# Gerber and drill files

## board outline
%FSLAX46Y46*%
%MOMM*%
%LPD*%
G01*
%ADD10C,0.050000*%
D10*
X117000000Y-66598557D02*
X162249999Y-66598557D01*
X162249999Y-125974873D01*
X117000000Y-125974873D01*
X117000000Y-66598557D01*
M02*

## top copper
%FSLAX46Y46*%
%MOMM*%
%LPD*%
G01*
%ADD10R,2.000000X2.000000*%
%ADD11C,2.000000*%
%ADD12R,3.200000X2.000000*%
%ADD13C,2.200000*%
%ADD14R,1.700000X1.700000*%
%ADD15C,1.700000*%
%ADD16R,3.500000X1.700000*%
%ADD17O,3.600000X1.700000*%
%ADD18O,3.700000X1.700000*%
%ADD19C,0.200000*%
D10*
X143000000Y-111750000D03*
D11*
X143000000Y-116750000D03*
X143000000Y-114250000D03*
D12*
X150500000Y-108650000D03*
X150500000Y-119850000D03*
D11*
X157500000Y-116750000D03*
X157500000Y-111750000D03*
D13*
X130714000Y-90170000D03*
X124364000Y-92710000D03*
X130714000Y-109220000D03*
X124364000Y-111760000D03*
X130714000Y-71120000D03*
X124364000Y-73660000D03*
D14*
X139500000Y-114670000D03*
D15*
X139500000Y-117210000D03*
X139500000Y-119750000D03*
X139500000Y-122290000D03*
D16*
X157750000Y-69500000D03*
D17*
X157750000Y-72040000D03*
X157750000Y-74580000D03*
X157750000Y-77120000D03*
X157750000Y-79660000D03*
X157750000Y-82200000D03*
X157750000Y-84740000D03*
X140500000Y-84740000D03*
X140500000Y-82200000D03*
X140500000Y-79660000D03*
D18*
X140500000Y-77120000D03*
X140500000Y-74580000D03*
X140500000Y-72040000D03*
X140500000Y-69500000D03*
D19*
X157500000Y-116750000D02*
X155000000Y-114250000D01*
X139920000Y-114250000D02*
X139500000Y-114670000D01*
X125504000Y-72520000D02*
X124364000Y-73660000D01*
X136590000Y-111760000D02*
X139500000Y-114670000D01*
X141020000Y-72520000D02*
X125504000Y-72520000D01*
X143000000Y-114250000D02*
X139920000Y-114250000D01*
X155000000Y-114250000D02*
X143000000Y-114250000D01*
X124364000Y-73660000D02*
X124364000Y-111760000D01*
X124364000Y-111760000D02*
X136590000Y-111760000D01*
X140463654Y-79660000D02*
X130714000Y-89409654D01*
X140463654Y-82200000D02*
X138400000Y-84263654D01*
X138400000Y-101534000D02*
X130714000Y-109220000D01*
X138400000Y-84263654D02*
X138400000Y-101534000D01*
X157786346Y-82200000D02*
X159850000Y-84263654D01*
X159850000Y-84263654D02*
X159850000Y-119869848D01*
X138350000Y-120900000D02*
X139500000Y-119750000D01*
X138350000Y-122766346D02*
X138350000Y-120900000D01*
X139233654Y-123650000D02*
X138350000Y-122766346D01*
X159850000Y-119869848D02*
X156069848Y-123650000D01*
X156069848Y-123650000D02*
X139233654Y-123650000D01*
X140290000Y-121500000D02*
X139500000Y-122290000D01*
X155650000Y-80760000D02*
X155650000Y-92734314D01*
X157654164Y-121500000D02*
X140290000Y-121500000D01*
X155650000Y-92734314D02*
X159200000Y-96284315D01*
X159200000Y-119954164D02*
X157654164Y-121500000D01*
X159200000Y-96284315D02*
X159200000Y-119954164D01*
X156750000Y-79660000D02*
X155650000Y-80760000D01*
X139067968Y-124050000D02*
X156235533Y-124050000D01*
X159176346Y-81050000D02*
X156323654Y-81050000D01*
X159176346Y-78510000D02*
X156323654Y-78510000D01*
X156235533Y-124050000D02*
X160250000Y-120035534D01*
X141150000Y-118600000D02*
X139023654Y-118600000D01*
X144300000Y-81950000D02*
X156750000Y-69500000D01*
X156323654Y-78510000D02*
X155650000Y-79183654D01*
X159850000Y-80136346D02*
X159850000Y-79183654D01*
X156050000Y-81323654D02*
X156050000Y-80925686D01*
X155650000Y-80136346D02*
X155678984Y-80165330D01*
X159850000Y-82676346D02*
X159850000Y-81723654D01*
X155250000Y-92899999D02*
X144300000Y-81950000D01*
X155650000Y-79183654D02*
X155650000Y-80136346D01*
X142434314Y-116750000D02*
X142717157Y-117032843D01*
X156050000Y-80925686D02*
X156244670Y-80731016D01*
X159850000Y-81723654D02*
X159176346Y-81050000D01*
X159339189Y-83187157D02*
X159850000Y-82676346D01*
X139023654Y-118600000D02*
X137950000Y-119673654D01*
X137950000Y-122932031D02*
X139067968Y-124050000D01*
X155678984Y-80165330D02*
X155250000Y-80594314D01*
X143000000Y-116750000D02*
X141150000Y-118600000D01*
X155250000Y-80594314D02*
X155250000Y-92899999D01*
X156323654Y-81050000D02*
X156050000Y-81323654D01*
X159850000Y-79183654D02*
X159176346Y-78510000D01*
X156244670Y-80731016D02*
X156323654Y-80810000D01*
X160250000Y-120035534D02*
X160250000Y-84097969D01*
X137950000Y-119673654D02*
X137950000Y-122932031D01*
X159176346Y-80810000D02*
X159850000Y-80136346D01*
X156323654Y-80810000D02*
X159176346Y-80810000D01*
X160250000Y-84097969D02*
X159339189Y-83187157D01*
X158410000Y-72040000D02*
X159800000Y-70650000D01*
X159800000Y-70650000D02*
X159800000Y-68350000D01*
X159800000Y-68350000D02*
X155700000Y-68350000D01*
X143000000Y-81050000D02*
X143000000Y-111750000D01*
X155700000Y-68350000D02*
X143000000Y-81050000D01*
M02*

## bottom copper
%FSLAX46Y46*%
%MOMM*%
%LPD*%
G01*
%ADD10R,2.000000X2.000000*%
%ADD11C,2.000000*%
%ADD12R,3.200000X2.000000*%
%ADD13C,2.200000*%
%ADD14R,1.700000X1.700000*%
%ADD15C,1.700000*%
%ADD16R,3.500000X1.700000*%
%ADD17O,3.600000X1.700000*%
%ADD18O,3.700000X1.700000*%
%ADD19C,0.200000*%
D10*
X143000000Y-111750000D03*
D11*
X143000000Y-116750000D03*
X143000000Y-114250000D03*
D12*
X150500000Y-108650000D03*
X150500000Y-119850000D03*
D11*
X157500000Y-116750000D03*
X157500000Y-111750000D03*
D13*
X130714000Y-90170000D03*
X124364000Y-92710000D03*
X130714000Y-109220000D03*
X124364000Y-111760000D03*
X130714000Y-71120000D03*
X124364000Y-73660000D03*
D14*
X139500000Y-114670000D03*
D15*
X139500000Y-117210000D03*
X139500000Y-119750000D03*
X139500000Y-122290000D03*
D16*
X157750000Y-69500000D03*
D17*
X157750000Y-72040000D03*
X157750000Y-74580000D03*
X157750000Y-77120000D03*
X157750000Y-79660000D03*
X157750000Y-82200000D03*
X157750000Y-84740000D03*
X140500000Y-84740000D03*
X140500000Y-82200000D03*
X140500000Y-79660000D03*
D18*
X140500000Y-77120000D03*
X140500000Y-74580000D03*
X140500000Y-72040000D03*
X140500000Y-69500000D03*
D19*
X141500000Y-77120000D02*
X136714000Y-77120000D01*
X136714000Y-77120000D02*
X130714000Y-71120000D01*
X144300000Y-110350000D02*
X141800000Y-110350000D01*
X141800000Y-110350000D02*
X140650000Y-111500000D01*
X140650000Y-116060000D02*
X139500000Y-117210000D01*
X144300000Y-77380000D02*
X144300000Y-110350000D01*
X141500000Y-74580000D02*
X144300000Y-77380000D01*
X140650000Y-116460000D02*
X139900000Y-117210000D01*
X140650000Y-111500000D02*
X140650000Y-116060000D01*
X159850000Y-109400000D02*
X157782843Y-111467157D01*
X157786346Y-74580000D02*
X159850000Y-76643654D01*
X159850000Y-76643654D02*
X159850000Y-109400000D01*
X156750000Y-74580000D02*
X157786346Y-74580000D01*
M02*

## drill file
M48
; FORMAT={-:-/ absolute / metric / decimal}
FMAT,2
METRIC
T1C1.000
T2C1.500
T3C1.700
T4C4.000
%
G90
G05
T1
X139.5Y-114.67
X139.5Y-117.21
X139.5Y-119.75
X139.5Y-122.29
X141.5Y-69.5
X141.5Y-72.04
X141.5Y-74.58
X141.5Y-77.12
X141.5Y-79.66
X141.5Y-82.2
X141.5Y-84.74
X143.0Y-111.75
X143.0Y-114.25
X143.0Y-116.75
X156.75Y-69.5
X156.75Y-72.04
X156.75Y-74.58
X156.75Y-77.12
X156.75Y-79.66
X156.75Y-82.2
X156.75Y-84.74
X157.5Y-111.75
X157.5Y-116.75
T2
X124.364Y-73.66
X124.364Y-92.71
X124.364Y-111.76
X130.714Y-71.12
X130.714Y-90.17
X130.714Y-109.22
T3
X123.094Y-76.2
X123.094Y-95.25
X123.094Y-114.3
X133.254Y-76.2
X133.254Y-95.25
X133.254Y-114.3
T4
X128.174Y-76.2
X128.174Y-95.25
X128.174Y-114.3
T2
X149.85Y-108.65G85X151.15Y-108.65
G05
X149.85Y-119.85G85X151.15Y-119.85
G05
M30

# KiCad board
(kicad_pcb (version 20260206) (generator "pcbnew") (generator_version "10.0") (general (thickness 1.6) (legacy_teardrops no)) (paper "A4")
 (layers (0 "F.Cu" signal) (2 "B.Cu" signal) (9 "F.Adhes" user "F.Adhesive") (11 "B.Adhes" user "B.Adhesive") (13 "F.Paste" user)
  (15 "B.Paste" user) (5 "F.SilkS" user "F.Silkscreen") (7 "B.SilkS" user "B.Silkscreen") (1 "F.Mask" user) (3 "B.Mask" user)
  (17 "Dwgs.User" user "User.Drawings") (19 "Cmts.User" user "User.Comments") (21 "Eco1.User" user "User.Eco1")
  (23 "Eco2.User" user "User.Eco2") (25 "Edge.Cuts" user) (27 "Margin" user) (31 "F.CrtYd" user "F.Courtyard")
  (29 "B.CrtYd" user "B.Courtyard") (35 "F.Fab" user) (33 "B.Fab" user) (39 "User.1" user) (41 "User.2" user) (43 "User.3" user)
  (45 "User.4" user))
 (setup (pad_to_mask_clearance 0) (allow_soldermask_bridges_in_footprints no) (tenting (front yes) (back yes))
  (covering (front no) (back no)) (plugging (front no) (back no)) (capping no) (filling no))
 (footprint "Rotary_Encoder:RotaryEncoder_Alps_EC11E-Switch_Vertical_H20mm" (layer "F.Cu") (at 143 111.75)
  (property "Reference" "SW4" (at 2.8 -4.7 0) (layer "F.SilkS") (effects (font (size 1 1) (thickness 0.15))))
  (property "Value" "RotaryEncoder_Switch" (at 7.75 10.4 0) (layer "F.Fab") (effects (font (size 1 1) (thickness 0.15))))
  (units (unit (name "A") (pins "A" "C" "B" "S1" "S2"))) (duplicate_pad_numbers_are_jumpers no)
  (pad "A" thru_hole rect (at 0 0) (size 2 2) (drill 1) (layers "*.Cu" "*.Mask") (remove_unused_layers no) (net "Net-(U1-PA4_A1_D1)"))
  (pad "B" thru_hole circle (at 0 5) (size 2 2) (drill 1) (layers "*.Cu" "*.Mask") (remove_unused_layers no) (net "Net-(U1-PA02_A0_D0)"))
  (pad "C" thru_hole circle (at 0 2.5) (size 2 2) (drill 1) (layers "*.Cu" "*.Mask") (remove_unused_layers no) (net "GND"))
  (pad "MP" thru_hole rect (at 7.5 -3.1) (size 3.2 2) (drill oval 2.8 1.5) (layers "*.Cu" "*.Mask") (remove_unused_layers no))
  (pad "MP" thru_hole rect (at 7.5 8.1) (size 3.2 2) (drill oval 2.8 1.5) (layers "*.Cu" "*.Mask") (remove_unused_layers no))
  (pad "S1" thru_hole circle (at 14.5 5) (size 2 2) (drill 1) (layers "*.Cu" "*.Mask") (remove_unused_layers no) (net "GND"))
  (pad "S2" thru_hole circle (at 14.5 0) (size 2 2) (drill 1) (layers "*.Cu" "*.Mask") (remove_unused_layers no) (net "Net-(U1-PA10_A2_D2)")))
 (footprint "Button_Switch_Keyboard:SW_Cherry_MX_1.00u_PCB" (layer "F.Cu") (at 130.714 90.17)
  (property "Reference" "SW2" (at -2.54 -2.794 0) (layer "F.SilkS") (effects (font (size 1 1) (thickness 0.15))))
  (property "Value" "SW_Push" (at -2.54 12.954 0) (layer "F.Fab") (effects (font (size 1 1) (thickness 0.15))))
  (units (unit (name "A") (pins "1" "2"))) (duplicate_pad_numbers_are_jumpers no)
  (pad "" np_thru_hole circle (at -7.62 5.08) (size 1.7 1.7) (drill 1.7) (layers "*.Cu" "*.Mask"))
  (pad "" np_thru_hole circle (at -2.54 5.08) (size 4 4) (drill 4) (layers "*.Cu" "*.Mask"))
  (pad "" np_thru_hole circle (at 2.54 5.08) (size 1.7 1.7) (drill 1.7) (layers "*.Cu" "*.Mask"))
  (pad "1" thru_hole circle (at 0 0) (size 2.2 2.2) (drill 1.5) (layers "*.Cu" "*.Mask") (remove_unused_layers no)
   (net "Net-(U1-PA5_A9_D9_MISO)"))
  (pad "2" thru_hole circle (at -6.35 2.54) (size 2.2 2.2) (drill 1.5) (layers "*.Cu" "*.Mask") (remove_unused_layers no) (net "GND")))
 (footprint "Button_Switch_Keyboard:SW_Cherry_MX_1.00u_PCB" (layer "F.Cu") (at 130.714 109.22)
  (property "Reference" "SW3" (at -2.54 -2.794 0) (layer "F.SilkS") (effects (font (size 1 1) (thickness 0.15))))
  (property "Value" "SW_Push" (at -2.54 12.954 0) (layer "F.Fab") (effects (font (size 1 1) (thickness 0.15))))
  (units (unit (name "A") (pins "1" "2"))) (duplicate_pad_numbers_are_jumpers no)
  (pad "" np_thru_hole circle (at -7.62 5.08) (size 1.7 1.7) (drill 1.7) (layers "*.Cu" "*.Mask"))
  (pad "" np_thru_hole circle (at -2.54 5.08) (size 4 4) (drill 4) (layers "*.Cu" "*.Mask"))
  (pad "" np_thru_hole circle (at 2.54 5.08) (size 1.7 1.7) (drill 1.7) (layers "*.Cu" "*.Mask"))
  (pad "1" thru_hole circle (at 0 0) (size 2.2 2.2) (drill 1.5) (layers "*.Cu" "*.Mask") (remove_unused_layers no)
   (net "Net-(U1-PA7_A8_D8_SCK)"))
  (pad "2" thru_hole circle (at -6.35 2.54) (size 2.2 2.2) (drill 1.5) (layers "*.Cu" "*.Mask") (remove_unused_layers no) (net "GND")))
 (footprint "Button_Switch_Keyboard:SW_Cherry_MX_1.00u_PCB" (layer "F.Cu") (at 130.714 71.12)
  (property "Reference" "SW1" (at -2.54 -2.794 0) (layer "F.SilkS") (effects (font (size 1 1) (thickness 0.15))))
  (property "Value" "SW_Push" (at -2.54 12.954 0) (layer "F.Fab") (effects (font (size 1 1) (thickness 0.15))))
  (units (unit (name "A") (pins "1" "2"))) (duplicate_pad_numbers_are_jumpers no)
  (pad "" np_thru_hole circle (at -7.62 5.08) (size 1.7 1.7) (drill 1.7) (layers "*.Cu" "*.Mask"))
  (pad "" np_thru_hole circle (at -2.54 5.08) (size 4 4) (drill 4) (layers "*.Cu" "*.Mask"))
  (pad "" np_thru_hole circle (at 2.54 5.08) (size 1.7 1.7) (drill 1.7) (layers "*.Cu" "*.Mask"))
  (pad "1" thru_hole circle (at 0 0) (size 2.2 2.2) (drill 1.5) (layers "*.Cu" "*.Mask") (remove_unused_layers no)
   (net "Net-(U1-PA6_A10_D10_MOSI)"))
  (pad "2" thru_hole circle (at -6.35 2.54) (size 2.2 2.2) (drill 1.5) (layers "*.Cu" "*.Mask") (remove_unused_layers no) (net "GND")))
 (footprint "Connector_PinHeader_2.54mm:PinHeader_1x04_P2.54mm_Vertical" (layer "F.Cu") (at 139.5 114.67)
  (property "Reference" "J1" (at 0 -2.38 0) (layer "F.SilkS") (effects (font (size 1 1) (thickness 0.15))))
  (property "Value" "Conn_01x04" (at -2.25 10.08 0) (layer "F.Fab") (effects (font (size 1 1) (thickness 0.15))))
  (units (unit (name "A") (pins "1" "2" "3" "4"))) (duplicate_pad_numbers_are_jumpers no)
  (pad "1" thru_hole rect (at 0 0) (size 1.7 1.7) (drill 1) (layers "*.Cu" "*.Mask") (remove_unused_layers no) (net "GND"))
  (pad "2" thru_hole circle (at 0 2.54) (size 1.7 1.7) (drill 1) (layers "*.Cu" "*.Mask") (remove_unused_layers no) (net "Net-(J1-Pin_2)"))
  (pad "3" thru_hole circle (at 0 5.08) (size 1.7 1.7) (drill 1) (layers "*.Cu" "*.Mask") (remove_unused_layers no) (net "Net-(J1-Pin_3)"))
  (pad "4" thru_hole circle (at 0 7.62) (size 1.7 1.7) (drill 1) (layers "*.Cu" "*.Mask") (remove_unused_layers no) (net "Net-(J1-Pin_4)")))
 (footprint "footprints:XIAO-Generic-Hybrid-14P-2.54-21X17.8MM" (layer "B.Cu") (at 149.125 77.12 180)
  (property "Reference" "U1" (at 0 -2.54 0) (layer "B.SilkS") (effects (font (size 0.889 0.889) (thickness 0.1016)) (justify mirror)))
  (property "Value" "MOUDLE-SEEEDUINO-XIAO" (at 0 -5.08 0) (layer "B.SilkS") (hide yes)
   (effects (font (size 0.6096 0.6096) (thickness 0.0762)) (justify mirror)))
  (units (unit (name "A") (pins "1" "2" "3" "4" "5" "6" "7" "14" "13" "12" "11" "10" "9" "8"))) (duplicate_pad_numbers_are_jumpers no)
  (pad "1" thru_hole rect (at -7.625 7.62 180) (size 3.5 1.7) (drill 1 (offset -1 0)) (layers "*.Cu" "*.Mask") (remove_unused_layers no)
   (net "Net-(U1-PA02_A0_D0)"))
  (pad "2" thru_hole oval (at -7.625 5.08 180) (size 3.6 1.7) (drill 1 (offset -1 0)) (layers "*.Cu" "*.Mask") (remove_unused_layers no)
   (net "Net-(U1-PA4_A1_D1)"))
  (pad "3" thru_hole oval (at -7.625 2.54 180) (size 3.6 1.7) (drill 1 (offset -1 0)) (layers "*.Cu" "*.Mask") (remove_unused_layers no)
   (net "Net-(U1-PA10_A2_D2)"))
  (pad "4" thru_hole oval (at -7.625 0 180) (size 3.6 1.7) (drill 1 (offset -1 0)) (layers "*.Cu" "*.Mask") (remove_unused_layers no)
   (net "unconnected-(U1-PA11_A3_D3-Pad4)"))
  (pad "5" thru_hole oval (at -7.625 -2.54 180) (size 3.6 1.7) (drill 1 (offset -1 0)) (layers "*.Cu" "*.Mask") (remove_unused_layers no)
   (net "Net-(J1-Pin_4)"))
  (pad "6" thru_hole oval (at -7.625 -5.08) (size 3.6 1.7) (drill 1 (offset 1 0)) (layers "*.Cu" "*.Mask") (remove_unused_layers no)
   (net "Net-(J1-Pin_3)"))
  (pad "7" thru_hole oval (at -7.625 -7.62 180) (size 3.6 1.7) (drill 1 (offset -1 0)) (layers "*.Cu" "*.Mask") (remove_unused_layers no)
   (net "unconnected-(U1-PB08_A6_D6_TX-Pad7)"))
  (pad "8" thru_hole oval (at 7.625 -7.62 180) (size 3.6 1.7) (drill 1 (offset 1 0)) (layers "*.Cu" "*.Mask") (remove_unused_layers no)
   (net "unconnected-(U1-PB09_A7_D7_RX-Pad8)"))
  (pad "9" thru_hole oval (at 7.625 -5.08 180) (size 3.6 1.7) (drill 1 (offset 1 0)) (layers "*.Cu" "*.Mask") (remove_unused_layers no)
   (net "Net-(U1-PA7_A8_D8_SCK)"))
  (pad "10" thru_hole oval (at 7.625 -2.54 180) (size 3.6 1.7) (drill 1 (offset 1 0)) (layers "*.Cu" "*.Mask") (remove_unused_layers no)
   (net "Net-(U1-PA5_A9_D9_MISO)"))
  (pad "11" thru_hole oval (at 7.625 0 180) (size 3.7 1.7) (drill 1 (offset 1 0)) (layers "*.Cu" "*.Mask") (remove_unused_layers no)
   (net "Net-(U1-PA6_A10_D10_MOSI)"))
  (pad "12" thru_hole oval (at 7.625 2.54 180) (size 3.7 1.7) (drill 1 (offset 1 0)) (layers "*.Cu" "*.Mask") (remove_unused_layers no)
   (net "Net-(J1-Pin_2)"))
  (pad "13" thru_hole oval (at 7.625 5.08 180) (size 3.7 1.7) (drill 1 (offset 1 0)) (layers "*.Cu" "*.Mask") (remove_unused_layers no)
   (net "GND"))
  (pad "14" thru_hole oval (at 7.625 7.62 180) (size 3.7 1.7) (drill 1 (offset 1 0)) (layers "*.Cu" "*.Mask") (remove_unused_layers no)
   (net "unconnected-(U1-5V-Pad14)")))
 (gr_rect (start 117 66.598557) (end 162.249999 125.974873) (stroke (width 0.05) (type default)) (fill no) (layer "Edge.Cuts"))
 (segment (start 141.5 77.12) (end 136.714 77.12) (width 0.2) (layer "B.Cu") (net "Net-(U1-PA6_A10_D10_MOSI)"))
 (segment (start 136.714 77.12) (end 130.714 71.12) (width 0.2) (layer "B.Cu") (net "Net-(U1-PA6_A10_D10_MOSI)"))
 (segment (start 157.5 116.75) (end 155 114.25) (width 0.2) (layer "F.Cu") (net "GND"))
 (segment (start 139.92 114.25) (end 139.5 114.67) (width 0.2) (layer "F.Cu") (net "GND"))
 (segment (start 125.504 72.52) (end 124.364 73.66) (width 0.2) (layer "F.Cu") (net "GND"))
 (segment (start 136.59 111.76) (end 139.5 114.67) (width 0.2) (layer "F.Cu") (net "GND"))
 (segment (start 141.02 72.52) (end 125.504 72.52) (width 0.2) (layer "F.Cu") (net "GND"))
 (segment (start 143 114.25) (end 139.92 114.25) (width 0.2) (layer "F.Cu") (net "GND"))
 (segment (start 155 114.25) (end 143 114.25) (width 0.2) (layer "F.Cu") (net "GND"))
 (segment (start 124.364 73.66) (end 124.364 111.76) (width 0.2) (layer "F.Cu") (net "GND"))
 (segment (start 124.364 111.76) (end 136.59 111.76) (width 0.2) (layer "F.Cu") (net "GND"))
 (segment (start 140.463654 79.66) (end 130.714 89.409654) (width 0.2) (layer "F.Cu") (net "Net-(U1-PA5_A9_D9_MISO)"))
 (segment (start 140.463654 82.2) (end 138.4 84.263654) (width 0.2) (layer "F.Cu") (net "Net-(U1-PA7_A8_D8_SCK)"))
 (segment (start 138.4 101.534) (end 130.714 109.22) (width 0.2) (layer "F.Cu") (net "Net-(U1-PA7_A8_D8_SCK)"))
 (segment (start 138.4 84.263654) (end 138.4 101.534) (width 0.2) (layer "F.Cu") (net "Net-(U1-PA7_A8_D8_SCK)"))
 (segment (start 157.786346 82.2) (end 159.85 84.263654) (width 0.2) (layer "F.Cu") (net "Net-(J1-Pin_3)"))
 (segment (start 159.85 84.263654) (end 159.85 119.869848) (width 0.2) (layer "F.Cu") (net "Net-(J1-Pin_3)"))
 (segment (start 138.35 120.9) (end 139.5 119.75) (width 0.2) (layer "F.Cu") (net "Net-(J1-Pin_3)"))
 (segment (start 138.35 122.766346) (end 138.35 120.9) (width 0.2) (layer "F.Cu") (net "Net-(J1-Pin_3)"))
 (segment (start 139.233654 123.65) (end 138.35 122.766346) (width 0.2) (layer "F.Cu") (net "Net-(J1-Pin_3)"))
 (segment (start 159.85 119.869848) (end 156.069848 123.65) (width 0.2) (layer "F.Cu") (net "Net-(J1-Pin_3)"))
 (segment (start 156.069848 123.65) (end 139.233654 123.65) (width 0.2) (layer "F.Cu") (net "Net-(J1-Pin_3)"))
 (segment (start 140.29 121.5) (end 139.5 122.29) (width 0.2) (layer "F.Cu") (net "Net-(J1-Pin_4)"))
 (segment (start 155.65 80.76) (end 155.65 92.734314) (width 0.2) (layer "F.Cu") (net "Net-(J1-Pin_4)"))
 (segment (start 157.654164 121.5) (end 140.29 121.5) (width 0.2) (layer "F.Cu") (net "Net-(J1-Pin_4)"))
 (segment (start 155.65 92.734314) (end 159.2 96.284315) (width 0.2) (layer "F.Cu") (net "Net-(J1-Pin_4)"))
 (segment (start 159.2 119.954164) (end 157.654164 121.5) (width 0.2) (layer "F.Cu") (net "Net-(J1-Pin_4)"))
 (segment (start 159.2 96.284315) (end 159.2 119.954164) (width 0.2) (layer "F.Cu") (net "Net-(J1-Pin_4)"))
 (segment (start 156.75 79.66) (end 155.65 80.76) (width 0.2) (layer "F.Cu") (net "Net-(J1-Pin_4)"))
 (segment (start 144.3 110.35) (end 141.8 110.35) (width 0.2) (layer "B.Cu") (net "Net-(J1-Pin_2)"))
 (segment (start 141.8 110.35) (end 140.65 111.5) (width 0.2) (layer "B.Cu") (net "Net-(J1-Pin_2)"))
 (segment (start 140.65 116.06) (end 139.5 117.21) (width 0.2) (layer "B.Cu") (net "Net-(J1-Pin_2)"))
 (segment (start 144.3 77.38) (end 144.3 110.35) (width 0.2) (layer "B.Cu") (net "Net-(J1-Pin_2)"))
 (segment (start 141.5 74.58) (end 144.3 77.38) (width 0.2) (layer "B.Cu") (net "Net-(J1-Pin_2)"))
 (segment (start 140.65 116.46) (end 139.9 117.21) (width 0.2) (layer "B.Cu") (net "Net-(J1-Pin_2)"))
 (segment (start 140.65 111.5) (end 140.65 116.06) (width 0.2) (layer "B.Cu") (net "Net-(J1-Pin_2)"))
 (segment (start 139.067968 124.05) (end 156.235533 124.05) (width 0.2) (layer "F.Cu") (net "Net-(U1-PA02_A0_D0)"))
 (segment (start 159.176346 81.05) (end 156.323654 81.05) (width 0.2) (layer "F.Cu") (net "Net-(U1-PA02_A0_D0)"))
 (segment (start 159.176346 78.51) (end 156.323654 78.51) (width 0.2) (layer "F.Cu") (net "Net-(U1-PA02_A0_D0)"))
 (segment (start 156.235533 124.05) (end 160.25 120.035534) (width 0.2) (layer "F.Cu") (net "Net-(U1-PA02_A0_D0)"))
 (segment (start 141.15 118.6) (end 139.023654 118.6) (width 0.2) (layer "F.Cu") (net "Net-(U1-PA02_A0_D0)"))
 (segment (start 144.3 81.95) (end 156.75 69.5) (width 0.2) (layer "F.Cu") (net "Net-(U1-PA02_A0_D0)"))
 (segment (start 156.323654 78.51) (end 155.65 79.183654) (width 0.2) (layer "F.Cu") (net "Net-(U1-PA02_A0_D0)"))
 (segment (start 159.85 80.136346) (end 159.85 79.183654) (width 0.2) (layer "F.Cu") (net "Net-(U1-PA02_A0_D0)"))
 (segment (start 156.05 81.323654) (end 156.05 80.925686) (width 0.2) (layer "F.Cu") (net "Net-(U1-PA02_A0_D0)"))
 (segment (start 155.65 80.136346) (end 155.678984 80.16533) (width 0.2) (layer "F.Cu") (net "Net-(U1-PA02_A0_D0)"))
 (segment (start 159.85 82.676346) (end 159.85 81.723654) (width 0.2) (layer "F.Cu") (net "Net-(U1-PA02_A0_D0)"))
 (segment (start 155.25 92.899999) (end 144.3 81.95) (width 0.2) (layer "F.Cu") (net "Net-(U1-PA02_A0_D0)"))
 (segment (start 155.65 79.183654) (end 155.65 80.136346) (width 0.2) (layer "F.Cu") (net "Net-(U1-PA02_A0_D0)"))
 (segment (start 142.434314 116.75) (end 142.717157 117.032843) (width 0.2) (layer "F.Cu") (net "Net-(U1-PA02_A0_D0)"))
 (segment (start 156.05 80.925686) (end 156.24467 80.731016) (width 0.2) (layer "F.Cu") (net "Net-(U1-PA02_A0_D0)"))
 (segment (start 159.85 81.723654) (end 159.176346 81.05) (width 0.2) (layer "F.Cu") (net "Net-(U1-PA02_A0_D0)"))
 (segment (start 159.339189 83.187157) (end 159.85 82.676346) (width 0.2) (layer "F.Cu") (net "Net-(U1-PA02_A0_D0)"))
 (segment (start 139.023654 118.6) (end 137.95 119.673654) (width 0.2) (layer "F.Cu") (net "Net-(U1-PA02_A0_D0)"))
 (segment (start 137.95 122.932031) (end 139.067968 124.05) (width 0.2) (layer "F.Cu") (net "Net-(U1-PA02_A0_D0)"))
 (segment (start 155.678984 80.16533) (end 155.25 80.594314) (width 0.2) (layer "F.Cu") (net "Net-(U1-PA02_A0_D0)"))
 (segment (start 143 116.75) (end 141.15 118.6) (width 0.2) (layer "F.Cu") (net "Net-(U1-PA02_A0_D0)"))
 (segment (start 155.25 80.594314) (end 155.25 92.899999) (width 0.2) (layer "F.Cu") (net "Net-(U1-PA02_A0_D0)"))
 (segment (start 156.323654 81.05) (end 156.05 81.323654) (width 0.2) (layer "F.Cu") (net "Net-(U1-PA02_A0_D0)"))
 (segment (start 159.85 79.183654) (end 159.176346 78.51) (width 0.2) (layer "F.Cu") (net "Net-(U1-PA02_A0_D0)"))
 (segment (start 156.24467 80.731016) (end 156.323654 80.81) (width 0.2) (layer "F.Cu") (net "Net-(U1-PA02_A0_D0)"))
 (segment (start 160.25 120.035534) (end 160.25 84.097969) (width 0.2) (layer "F.Cu") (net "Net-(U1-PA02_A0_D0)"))
 (segment (start 137.95 119.673654) (end 137.95 122.932031) (width 0.2) (layer "F.Cu") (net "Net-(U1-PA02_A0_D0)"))
 (segment (start 159.176346 80.81) (end 159.85 80.136346) (width 0.2) (layer "F.Cu") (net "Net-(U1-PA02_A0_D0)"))
 (segment (start 156.323654 80.81) (end 159.176346 80.81) (width 0.2) (layer "F.Cu") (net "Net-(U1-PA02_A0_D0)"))
 (segment (start 160.25 84.097969) (end 159.339189 83.187157) (width 0.2) (layer "F.Cu") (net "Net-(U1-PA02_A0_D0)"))
 (segment (start 158.41 72.04) (end 159.8 70.65) (width 0.2) (layer "F.Cu") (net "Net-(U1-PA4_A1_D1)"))
 (segment (start 159.8 70.65) (end 159.8 68.35) (width 0.2) (layer "F.Cu") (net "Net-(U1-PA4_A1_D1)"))
 (segment (start 159.8 68.35) (end 155.7 68.35) (width 0.2) (layer "F.Cu") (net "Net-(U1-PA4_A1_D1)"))
 (segment (start 143 81.05) (end 143 111.75) (width 0.2) (layer "F.Cu") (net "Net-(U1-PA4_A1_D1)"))
 (segment (start 155.7 68.35) (end 143 81.05) (width 0.2) (layer "F.Cu") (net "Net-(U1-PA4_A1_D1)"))
 (segment (start 159.85 109.4) (end 157.782843 111.467157) (width 0.2) (layer "B.Cu") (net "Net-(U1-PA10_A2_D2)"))
 (segment (start 157.786346 74.58) (end 159.85 76.643654) (width 0.2) (layer "B.Cu") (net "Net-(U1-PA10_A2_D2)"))
 (segment (start 159.85 76.643654) (end 159.85 109.4) (width 0.2) (layer "B.Cu") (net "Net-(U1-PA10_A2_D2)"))
 (segment (start 156.75 74.58) (end 157.786346 74.58) (width 0.2) (layer "B.Cu") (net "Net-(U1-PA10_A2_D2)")))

